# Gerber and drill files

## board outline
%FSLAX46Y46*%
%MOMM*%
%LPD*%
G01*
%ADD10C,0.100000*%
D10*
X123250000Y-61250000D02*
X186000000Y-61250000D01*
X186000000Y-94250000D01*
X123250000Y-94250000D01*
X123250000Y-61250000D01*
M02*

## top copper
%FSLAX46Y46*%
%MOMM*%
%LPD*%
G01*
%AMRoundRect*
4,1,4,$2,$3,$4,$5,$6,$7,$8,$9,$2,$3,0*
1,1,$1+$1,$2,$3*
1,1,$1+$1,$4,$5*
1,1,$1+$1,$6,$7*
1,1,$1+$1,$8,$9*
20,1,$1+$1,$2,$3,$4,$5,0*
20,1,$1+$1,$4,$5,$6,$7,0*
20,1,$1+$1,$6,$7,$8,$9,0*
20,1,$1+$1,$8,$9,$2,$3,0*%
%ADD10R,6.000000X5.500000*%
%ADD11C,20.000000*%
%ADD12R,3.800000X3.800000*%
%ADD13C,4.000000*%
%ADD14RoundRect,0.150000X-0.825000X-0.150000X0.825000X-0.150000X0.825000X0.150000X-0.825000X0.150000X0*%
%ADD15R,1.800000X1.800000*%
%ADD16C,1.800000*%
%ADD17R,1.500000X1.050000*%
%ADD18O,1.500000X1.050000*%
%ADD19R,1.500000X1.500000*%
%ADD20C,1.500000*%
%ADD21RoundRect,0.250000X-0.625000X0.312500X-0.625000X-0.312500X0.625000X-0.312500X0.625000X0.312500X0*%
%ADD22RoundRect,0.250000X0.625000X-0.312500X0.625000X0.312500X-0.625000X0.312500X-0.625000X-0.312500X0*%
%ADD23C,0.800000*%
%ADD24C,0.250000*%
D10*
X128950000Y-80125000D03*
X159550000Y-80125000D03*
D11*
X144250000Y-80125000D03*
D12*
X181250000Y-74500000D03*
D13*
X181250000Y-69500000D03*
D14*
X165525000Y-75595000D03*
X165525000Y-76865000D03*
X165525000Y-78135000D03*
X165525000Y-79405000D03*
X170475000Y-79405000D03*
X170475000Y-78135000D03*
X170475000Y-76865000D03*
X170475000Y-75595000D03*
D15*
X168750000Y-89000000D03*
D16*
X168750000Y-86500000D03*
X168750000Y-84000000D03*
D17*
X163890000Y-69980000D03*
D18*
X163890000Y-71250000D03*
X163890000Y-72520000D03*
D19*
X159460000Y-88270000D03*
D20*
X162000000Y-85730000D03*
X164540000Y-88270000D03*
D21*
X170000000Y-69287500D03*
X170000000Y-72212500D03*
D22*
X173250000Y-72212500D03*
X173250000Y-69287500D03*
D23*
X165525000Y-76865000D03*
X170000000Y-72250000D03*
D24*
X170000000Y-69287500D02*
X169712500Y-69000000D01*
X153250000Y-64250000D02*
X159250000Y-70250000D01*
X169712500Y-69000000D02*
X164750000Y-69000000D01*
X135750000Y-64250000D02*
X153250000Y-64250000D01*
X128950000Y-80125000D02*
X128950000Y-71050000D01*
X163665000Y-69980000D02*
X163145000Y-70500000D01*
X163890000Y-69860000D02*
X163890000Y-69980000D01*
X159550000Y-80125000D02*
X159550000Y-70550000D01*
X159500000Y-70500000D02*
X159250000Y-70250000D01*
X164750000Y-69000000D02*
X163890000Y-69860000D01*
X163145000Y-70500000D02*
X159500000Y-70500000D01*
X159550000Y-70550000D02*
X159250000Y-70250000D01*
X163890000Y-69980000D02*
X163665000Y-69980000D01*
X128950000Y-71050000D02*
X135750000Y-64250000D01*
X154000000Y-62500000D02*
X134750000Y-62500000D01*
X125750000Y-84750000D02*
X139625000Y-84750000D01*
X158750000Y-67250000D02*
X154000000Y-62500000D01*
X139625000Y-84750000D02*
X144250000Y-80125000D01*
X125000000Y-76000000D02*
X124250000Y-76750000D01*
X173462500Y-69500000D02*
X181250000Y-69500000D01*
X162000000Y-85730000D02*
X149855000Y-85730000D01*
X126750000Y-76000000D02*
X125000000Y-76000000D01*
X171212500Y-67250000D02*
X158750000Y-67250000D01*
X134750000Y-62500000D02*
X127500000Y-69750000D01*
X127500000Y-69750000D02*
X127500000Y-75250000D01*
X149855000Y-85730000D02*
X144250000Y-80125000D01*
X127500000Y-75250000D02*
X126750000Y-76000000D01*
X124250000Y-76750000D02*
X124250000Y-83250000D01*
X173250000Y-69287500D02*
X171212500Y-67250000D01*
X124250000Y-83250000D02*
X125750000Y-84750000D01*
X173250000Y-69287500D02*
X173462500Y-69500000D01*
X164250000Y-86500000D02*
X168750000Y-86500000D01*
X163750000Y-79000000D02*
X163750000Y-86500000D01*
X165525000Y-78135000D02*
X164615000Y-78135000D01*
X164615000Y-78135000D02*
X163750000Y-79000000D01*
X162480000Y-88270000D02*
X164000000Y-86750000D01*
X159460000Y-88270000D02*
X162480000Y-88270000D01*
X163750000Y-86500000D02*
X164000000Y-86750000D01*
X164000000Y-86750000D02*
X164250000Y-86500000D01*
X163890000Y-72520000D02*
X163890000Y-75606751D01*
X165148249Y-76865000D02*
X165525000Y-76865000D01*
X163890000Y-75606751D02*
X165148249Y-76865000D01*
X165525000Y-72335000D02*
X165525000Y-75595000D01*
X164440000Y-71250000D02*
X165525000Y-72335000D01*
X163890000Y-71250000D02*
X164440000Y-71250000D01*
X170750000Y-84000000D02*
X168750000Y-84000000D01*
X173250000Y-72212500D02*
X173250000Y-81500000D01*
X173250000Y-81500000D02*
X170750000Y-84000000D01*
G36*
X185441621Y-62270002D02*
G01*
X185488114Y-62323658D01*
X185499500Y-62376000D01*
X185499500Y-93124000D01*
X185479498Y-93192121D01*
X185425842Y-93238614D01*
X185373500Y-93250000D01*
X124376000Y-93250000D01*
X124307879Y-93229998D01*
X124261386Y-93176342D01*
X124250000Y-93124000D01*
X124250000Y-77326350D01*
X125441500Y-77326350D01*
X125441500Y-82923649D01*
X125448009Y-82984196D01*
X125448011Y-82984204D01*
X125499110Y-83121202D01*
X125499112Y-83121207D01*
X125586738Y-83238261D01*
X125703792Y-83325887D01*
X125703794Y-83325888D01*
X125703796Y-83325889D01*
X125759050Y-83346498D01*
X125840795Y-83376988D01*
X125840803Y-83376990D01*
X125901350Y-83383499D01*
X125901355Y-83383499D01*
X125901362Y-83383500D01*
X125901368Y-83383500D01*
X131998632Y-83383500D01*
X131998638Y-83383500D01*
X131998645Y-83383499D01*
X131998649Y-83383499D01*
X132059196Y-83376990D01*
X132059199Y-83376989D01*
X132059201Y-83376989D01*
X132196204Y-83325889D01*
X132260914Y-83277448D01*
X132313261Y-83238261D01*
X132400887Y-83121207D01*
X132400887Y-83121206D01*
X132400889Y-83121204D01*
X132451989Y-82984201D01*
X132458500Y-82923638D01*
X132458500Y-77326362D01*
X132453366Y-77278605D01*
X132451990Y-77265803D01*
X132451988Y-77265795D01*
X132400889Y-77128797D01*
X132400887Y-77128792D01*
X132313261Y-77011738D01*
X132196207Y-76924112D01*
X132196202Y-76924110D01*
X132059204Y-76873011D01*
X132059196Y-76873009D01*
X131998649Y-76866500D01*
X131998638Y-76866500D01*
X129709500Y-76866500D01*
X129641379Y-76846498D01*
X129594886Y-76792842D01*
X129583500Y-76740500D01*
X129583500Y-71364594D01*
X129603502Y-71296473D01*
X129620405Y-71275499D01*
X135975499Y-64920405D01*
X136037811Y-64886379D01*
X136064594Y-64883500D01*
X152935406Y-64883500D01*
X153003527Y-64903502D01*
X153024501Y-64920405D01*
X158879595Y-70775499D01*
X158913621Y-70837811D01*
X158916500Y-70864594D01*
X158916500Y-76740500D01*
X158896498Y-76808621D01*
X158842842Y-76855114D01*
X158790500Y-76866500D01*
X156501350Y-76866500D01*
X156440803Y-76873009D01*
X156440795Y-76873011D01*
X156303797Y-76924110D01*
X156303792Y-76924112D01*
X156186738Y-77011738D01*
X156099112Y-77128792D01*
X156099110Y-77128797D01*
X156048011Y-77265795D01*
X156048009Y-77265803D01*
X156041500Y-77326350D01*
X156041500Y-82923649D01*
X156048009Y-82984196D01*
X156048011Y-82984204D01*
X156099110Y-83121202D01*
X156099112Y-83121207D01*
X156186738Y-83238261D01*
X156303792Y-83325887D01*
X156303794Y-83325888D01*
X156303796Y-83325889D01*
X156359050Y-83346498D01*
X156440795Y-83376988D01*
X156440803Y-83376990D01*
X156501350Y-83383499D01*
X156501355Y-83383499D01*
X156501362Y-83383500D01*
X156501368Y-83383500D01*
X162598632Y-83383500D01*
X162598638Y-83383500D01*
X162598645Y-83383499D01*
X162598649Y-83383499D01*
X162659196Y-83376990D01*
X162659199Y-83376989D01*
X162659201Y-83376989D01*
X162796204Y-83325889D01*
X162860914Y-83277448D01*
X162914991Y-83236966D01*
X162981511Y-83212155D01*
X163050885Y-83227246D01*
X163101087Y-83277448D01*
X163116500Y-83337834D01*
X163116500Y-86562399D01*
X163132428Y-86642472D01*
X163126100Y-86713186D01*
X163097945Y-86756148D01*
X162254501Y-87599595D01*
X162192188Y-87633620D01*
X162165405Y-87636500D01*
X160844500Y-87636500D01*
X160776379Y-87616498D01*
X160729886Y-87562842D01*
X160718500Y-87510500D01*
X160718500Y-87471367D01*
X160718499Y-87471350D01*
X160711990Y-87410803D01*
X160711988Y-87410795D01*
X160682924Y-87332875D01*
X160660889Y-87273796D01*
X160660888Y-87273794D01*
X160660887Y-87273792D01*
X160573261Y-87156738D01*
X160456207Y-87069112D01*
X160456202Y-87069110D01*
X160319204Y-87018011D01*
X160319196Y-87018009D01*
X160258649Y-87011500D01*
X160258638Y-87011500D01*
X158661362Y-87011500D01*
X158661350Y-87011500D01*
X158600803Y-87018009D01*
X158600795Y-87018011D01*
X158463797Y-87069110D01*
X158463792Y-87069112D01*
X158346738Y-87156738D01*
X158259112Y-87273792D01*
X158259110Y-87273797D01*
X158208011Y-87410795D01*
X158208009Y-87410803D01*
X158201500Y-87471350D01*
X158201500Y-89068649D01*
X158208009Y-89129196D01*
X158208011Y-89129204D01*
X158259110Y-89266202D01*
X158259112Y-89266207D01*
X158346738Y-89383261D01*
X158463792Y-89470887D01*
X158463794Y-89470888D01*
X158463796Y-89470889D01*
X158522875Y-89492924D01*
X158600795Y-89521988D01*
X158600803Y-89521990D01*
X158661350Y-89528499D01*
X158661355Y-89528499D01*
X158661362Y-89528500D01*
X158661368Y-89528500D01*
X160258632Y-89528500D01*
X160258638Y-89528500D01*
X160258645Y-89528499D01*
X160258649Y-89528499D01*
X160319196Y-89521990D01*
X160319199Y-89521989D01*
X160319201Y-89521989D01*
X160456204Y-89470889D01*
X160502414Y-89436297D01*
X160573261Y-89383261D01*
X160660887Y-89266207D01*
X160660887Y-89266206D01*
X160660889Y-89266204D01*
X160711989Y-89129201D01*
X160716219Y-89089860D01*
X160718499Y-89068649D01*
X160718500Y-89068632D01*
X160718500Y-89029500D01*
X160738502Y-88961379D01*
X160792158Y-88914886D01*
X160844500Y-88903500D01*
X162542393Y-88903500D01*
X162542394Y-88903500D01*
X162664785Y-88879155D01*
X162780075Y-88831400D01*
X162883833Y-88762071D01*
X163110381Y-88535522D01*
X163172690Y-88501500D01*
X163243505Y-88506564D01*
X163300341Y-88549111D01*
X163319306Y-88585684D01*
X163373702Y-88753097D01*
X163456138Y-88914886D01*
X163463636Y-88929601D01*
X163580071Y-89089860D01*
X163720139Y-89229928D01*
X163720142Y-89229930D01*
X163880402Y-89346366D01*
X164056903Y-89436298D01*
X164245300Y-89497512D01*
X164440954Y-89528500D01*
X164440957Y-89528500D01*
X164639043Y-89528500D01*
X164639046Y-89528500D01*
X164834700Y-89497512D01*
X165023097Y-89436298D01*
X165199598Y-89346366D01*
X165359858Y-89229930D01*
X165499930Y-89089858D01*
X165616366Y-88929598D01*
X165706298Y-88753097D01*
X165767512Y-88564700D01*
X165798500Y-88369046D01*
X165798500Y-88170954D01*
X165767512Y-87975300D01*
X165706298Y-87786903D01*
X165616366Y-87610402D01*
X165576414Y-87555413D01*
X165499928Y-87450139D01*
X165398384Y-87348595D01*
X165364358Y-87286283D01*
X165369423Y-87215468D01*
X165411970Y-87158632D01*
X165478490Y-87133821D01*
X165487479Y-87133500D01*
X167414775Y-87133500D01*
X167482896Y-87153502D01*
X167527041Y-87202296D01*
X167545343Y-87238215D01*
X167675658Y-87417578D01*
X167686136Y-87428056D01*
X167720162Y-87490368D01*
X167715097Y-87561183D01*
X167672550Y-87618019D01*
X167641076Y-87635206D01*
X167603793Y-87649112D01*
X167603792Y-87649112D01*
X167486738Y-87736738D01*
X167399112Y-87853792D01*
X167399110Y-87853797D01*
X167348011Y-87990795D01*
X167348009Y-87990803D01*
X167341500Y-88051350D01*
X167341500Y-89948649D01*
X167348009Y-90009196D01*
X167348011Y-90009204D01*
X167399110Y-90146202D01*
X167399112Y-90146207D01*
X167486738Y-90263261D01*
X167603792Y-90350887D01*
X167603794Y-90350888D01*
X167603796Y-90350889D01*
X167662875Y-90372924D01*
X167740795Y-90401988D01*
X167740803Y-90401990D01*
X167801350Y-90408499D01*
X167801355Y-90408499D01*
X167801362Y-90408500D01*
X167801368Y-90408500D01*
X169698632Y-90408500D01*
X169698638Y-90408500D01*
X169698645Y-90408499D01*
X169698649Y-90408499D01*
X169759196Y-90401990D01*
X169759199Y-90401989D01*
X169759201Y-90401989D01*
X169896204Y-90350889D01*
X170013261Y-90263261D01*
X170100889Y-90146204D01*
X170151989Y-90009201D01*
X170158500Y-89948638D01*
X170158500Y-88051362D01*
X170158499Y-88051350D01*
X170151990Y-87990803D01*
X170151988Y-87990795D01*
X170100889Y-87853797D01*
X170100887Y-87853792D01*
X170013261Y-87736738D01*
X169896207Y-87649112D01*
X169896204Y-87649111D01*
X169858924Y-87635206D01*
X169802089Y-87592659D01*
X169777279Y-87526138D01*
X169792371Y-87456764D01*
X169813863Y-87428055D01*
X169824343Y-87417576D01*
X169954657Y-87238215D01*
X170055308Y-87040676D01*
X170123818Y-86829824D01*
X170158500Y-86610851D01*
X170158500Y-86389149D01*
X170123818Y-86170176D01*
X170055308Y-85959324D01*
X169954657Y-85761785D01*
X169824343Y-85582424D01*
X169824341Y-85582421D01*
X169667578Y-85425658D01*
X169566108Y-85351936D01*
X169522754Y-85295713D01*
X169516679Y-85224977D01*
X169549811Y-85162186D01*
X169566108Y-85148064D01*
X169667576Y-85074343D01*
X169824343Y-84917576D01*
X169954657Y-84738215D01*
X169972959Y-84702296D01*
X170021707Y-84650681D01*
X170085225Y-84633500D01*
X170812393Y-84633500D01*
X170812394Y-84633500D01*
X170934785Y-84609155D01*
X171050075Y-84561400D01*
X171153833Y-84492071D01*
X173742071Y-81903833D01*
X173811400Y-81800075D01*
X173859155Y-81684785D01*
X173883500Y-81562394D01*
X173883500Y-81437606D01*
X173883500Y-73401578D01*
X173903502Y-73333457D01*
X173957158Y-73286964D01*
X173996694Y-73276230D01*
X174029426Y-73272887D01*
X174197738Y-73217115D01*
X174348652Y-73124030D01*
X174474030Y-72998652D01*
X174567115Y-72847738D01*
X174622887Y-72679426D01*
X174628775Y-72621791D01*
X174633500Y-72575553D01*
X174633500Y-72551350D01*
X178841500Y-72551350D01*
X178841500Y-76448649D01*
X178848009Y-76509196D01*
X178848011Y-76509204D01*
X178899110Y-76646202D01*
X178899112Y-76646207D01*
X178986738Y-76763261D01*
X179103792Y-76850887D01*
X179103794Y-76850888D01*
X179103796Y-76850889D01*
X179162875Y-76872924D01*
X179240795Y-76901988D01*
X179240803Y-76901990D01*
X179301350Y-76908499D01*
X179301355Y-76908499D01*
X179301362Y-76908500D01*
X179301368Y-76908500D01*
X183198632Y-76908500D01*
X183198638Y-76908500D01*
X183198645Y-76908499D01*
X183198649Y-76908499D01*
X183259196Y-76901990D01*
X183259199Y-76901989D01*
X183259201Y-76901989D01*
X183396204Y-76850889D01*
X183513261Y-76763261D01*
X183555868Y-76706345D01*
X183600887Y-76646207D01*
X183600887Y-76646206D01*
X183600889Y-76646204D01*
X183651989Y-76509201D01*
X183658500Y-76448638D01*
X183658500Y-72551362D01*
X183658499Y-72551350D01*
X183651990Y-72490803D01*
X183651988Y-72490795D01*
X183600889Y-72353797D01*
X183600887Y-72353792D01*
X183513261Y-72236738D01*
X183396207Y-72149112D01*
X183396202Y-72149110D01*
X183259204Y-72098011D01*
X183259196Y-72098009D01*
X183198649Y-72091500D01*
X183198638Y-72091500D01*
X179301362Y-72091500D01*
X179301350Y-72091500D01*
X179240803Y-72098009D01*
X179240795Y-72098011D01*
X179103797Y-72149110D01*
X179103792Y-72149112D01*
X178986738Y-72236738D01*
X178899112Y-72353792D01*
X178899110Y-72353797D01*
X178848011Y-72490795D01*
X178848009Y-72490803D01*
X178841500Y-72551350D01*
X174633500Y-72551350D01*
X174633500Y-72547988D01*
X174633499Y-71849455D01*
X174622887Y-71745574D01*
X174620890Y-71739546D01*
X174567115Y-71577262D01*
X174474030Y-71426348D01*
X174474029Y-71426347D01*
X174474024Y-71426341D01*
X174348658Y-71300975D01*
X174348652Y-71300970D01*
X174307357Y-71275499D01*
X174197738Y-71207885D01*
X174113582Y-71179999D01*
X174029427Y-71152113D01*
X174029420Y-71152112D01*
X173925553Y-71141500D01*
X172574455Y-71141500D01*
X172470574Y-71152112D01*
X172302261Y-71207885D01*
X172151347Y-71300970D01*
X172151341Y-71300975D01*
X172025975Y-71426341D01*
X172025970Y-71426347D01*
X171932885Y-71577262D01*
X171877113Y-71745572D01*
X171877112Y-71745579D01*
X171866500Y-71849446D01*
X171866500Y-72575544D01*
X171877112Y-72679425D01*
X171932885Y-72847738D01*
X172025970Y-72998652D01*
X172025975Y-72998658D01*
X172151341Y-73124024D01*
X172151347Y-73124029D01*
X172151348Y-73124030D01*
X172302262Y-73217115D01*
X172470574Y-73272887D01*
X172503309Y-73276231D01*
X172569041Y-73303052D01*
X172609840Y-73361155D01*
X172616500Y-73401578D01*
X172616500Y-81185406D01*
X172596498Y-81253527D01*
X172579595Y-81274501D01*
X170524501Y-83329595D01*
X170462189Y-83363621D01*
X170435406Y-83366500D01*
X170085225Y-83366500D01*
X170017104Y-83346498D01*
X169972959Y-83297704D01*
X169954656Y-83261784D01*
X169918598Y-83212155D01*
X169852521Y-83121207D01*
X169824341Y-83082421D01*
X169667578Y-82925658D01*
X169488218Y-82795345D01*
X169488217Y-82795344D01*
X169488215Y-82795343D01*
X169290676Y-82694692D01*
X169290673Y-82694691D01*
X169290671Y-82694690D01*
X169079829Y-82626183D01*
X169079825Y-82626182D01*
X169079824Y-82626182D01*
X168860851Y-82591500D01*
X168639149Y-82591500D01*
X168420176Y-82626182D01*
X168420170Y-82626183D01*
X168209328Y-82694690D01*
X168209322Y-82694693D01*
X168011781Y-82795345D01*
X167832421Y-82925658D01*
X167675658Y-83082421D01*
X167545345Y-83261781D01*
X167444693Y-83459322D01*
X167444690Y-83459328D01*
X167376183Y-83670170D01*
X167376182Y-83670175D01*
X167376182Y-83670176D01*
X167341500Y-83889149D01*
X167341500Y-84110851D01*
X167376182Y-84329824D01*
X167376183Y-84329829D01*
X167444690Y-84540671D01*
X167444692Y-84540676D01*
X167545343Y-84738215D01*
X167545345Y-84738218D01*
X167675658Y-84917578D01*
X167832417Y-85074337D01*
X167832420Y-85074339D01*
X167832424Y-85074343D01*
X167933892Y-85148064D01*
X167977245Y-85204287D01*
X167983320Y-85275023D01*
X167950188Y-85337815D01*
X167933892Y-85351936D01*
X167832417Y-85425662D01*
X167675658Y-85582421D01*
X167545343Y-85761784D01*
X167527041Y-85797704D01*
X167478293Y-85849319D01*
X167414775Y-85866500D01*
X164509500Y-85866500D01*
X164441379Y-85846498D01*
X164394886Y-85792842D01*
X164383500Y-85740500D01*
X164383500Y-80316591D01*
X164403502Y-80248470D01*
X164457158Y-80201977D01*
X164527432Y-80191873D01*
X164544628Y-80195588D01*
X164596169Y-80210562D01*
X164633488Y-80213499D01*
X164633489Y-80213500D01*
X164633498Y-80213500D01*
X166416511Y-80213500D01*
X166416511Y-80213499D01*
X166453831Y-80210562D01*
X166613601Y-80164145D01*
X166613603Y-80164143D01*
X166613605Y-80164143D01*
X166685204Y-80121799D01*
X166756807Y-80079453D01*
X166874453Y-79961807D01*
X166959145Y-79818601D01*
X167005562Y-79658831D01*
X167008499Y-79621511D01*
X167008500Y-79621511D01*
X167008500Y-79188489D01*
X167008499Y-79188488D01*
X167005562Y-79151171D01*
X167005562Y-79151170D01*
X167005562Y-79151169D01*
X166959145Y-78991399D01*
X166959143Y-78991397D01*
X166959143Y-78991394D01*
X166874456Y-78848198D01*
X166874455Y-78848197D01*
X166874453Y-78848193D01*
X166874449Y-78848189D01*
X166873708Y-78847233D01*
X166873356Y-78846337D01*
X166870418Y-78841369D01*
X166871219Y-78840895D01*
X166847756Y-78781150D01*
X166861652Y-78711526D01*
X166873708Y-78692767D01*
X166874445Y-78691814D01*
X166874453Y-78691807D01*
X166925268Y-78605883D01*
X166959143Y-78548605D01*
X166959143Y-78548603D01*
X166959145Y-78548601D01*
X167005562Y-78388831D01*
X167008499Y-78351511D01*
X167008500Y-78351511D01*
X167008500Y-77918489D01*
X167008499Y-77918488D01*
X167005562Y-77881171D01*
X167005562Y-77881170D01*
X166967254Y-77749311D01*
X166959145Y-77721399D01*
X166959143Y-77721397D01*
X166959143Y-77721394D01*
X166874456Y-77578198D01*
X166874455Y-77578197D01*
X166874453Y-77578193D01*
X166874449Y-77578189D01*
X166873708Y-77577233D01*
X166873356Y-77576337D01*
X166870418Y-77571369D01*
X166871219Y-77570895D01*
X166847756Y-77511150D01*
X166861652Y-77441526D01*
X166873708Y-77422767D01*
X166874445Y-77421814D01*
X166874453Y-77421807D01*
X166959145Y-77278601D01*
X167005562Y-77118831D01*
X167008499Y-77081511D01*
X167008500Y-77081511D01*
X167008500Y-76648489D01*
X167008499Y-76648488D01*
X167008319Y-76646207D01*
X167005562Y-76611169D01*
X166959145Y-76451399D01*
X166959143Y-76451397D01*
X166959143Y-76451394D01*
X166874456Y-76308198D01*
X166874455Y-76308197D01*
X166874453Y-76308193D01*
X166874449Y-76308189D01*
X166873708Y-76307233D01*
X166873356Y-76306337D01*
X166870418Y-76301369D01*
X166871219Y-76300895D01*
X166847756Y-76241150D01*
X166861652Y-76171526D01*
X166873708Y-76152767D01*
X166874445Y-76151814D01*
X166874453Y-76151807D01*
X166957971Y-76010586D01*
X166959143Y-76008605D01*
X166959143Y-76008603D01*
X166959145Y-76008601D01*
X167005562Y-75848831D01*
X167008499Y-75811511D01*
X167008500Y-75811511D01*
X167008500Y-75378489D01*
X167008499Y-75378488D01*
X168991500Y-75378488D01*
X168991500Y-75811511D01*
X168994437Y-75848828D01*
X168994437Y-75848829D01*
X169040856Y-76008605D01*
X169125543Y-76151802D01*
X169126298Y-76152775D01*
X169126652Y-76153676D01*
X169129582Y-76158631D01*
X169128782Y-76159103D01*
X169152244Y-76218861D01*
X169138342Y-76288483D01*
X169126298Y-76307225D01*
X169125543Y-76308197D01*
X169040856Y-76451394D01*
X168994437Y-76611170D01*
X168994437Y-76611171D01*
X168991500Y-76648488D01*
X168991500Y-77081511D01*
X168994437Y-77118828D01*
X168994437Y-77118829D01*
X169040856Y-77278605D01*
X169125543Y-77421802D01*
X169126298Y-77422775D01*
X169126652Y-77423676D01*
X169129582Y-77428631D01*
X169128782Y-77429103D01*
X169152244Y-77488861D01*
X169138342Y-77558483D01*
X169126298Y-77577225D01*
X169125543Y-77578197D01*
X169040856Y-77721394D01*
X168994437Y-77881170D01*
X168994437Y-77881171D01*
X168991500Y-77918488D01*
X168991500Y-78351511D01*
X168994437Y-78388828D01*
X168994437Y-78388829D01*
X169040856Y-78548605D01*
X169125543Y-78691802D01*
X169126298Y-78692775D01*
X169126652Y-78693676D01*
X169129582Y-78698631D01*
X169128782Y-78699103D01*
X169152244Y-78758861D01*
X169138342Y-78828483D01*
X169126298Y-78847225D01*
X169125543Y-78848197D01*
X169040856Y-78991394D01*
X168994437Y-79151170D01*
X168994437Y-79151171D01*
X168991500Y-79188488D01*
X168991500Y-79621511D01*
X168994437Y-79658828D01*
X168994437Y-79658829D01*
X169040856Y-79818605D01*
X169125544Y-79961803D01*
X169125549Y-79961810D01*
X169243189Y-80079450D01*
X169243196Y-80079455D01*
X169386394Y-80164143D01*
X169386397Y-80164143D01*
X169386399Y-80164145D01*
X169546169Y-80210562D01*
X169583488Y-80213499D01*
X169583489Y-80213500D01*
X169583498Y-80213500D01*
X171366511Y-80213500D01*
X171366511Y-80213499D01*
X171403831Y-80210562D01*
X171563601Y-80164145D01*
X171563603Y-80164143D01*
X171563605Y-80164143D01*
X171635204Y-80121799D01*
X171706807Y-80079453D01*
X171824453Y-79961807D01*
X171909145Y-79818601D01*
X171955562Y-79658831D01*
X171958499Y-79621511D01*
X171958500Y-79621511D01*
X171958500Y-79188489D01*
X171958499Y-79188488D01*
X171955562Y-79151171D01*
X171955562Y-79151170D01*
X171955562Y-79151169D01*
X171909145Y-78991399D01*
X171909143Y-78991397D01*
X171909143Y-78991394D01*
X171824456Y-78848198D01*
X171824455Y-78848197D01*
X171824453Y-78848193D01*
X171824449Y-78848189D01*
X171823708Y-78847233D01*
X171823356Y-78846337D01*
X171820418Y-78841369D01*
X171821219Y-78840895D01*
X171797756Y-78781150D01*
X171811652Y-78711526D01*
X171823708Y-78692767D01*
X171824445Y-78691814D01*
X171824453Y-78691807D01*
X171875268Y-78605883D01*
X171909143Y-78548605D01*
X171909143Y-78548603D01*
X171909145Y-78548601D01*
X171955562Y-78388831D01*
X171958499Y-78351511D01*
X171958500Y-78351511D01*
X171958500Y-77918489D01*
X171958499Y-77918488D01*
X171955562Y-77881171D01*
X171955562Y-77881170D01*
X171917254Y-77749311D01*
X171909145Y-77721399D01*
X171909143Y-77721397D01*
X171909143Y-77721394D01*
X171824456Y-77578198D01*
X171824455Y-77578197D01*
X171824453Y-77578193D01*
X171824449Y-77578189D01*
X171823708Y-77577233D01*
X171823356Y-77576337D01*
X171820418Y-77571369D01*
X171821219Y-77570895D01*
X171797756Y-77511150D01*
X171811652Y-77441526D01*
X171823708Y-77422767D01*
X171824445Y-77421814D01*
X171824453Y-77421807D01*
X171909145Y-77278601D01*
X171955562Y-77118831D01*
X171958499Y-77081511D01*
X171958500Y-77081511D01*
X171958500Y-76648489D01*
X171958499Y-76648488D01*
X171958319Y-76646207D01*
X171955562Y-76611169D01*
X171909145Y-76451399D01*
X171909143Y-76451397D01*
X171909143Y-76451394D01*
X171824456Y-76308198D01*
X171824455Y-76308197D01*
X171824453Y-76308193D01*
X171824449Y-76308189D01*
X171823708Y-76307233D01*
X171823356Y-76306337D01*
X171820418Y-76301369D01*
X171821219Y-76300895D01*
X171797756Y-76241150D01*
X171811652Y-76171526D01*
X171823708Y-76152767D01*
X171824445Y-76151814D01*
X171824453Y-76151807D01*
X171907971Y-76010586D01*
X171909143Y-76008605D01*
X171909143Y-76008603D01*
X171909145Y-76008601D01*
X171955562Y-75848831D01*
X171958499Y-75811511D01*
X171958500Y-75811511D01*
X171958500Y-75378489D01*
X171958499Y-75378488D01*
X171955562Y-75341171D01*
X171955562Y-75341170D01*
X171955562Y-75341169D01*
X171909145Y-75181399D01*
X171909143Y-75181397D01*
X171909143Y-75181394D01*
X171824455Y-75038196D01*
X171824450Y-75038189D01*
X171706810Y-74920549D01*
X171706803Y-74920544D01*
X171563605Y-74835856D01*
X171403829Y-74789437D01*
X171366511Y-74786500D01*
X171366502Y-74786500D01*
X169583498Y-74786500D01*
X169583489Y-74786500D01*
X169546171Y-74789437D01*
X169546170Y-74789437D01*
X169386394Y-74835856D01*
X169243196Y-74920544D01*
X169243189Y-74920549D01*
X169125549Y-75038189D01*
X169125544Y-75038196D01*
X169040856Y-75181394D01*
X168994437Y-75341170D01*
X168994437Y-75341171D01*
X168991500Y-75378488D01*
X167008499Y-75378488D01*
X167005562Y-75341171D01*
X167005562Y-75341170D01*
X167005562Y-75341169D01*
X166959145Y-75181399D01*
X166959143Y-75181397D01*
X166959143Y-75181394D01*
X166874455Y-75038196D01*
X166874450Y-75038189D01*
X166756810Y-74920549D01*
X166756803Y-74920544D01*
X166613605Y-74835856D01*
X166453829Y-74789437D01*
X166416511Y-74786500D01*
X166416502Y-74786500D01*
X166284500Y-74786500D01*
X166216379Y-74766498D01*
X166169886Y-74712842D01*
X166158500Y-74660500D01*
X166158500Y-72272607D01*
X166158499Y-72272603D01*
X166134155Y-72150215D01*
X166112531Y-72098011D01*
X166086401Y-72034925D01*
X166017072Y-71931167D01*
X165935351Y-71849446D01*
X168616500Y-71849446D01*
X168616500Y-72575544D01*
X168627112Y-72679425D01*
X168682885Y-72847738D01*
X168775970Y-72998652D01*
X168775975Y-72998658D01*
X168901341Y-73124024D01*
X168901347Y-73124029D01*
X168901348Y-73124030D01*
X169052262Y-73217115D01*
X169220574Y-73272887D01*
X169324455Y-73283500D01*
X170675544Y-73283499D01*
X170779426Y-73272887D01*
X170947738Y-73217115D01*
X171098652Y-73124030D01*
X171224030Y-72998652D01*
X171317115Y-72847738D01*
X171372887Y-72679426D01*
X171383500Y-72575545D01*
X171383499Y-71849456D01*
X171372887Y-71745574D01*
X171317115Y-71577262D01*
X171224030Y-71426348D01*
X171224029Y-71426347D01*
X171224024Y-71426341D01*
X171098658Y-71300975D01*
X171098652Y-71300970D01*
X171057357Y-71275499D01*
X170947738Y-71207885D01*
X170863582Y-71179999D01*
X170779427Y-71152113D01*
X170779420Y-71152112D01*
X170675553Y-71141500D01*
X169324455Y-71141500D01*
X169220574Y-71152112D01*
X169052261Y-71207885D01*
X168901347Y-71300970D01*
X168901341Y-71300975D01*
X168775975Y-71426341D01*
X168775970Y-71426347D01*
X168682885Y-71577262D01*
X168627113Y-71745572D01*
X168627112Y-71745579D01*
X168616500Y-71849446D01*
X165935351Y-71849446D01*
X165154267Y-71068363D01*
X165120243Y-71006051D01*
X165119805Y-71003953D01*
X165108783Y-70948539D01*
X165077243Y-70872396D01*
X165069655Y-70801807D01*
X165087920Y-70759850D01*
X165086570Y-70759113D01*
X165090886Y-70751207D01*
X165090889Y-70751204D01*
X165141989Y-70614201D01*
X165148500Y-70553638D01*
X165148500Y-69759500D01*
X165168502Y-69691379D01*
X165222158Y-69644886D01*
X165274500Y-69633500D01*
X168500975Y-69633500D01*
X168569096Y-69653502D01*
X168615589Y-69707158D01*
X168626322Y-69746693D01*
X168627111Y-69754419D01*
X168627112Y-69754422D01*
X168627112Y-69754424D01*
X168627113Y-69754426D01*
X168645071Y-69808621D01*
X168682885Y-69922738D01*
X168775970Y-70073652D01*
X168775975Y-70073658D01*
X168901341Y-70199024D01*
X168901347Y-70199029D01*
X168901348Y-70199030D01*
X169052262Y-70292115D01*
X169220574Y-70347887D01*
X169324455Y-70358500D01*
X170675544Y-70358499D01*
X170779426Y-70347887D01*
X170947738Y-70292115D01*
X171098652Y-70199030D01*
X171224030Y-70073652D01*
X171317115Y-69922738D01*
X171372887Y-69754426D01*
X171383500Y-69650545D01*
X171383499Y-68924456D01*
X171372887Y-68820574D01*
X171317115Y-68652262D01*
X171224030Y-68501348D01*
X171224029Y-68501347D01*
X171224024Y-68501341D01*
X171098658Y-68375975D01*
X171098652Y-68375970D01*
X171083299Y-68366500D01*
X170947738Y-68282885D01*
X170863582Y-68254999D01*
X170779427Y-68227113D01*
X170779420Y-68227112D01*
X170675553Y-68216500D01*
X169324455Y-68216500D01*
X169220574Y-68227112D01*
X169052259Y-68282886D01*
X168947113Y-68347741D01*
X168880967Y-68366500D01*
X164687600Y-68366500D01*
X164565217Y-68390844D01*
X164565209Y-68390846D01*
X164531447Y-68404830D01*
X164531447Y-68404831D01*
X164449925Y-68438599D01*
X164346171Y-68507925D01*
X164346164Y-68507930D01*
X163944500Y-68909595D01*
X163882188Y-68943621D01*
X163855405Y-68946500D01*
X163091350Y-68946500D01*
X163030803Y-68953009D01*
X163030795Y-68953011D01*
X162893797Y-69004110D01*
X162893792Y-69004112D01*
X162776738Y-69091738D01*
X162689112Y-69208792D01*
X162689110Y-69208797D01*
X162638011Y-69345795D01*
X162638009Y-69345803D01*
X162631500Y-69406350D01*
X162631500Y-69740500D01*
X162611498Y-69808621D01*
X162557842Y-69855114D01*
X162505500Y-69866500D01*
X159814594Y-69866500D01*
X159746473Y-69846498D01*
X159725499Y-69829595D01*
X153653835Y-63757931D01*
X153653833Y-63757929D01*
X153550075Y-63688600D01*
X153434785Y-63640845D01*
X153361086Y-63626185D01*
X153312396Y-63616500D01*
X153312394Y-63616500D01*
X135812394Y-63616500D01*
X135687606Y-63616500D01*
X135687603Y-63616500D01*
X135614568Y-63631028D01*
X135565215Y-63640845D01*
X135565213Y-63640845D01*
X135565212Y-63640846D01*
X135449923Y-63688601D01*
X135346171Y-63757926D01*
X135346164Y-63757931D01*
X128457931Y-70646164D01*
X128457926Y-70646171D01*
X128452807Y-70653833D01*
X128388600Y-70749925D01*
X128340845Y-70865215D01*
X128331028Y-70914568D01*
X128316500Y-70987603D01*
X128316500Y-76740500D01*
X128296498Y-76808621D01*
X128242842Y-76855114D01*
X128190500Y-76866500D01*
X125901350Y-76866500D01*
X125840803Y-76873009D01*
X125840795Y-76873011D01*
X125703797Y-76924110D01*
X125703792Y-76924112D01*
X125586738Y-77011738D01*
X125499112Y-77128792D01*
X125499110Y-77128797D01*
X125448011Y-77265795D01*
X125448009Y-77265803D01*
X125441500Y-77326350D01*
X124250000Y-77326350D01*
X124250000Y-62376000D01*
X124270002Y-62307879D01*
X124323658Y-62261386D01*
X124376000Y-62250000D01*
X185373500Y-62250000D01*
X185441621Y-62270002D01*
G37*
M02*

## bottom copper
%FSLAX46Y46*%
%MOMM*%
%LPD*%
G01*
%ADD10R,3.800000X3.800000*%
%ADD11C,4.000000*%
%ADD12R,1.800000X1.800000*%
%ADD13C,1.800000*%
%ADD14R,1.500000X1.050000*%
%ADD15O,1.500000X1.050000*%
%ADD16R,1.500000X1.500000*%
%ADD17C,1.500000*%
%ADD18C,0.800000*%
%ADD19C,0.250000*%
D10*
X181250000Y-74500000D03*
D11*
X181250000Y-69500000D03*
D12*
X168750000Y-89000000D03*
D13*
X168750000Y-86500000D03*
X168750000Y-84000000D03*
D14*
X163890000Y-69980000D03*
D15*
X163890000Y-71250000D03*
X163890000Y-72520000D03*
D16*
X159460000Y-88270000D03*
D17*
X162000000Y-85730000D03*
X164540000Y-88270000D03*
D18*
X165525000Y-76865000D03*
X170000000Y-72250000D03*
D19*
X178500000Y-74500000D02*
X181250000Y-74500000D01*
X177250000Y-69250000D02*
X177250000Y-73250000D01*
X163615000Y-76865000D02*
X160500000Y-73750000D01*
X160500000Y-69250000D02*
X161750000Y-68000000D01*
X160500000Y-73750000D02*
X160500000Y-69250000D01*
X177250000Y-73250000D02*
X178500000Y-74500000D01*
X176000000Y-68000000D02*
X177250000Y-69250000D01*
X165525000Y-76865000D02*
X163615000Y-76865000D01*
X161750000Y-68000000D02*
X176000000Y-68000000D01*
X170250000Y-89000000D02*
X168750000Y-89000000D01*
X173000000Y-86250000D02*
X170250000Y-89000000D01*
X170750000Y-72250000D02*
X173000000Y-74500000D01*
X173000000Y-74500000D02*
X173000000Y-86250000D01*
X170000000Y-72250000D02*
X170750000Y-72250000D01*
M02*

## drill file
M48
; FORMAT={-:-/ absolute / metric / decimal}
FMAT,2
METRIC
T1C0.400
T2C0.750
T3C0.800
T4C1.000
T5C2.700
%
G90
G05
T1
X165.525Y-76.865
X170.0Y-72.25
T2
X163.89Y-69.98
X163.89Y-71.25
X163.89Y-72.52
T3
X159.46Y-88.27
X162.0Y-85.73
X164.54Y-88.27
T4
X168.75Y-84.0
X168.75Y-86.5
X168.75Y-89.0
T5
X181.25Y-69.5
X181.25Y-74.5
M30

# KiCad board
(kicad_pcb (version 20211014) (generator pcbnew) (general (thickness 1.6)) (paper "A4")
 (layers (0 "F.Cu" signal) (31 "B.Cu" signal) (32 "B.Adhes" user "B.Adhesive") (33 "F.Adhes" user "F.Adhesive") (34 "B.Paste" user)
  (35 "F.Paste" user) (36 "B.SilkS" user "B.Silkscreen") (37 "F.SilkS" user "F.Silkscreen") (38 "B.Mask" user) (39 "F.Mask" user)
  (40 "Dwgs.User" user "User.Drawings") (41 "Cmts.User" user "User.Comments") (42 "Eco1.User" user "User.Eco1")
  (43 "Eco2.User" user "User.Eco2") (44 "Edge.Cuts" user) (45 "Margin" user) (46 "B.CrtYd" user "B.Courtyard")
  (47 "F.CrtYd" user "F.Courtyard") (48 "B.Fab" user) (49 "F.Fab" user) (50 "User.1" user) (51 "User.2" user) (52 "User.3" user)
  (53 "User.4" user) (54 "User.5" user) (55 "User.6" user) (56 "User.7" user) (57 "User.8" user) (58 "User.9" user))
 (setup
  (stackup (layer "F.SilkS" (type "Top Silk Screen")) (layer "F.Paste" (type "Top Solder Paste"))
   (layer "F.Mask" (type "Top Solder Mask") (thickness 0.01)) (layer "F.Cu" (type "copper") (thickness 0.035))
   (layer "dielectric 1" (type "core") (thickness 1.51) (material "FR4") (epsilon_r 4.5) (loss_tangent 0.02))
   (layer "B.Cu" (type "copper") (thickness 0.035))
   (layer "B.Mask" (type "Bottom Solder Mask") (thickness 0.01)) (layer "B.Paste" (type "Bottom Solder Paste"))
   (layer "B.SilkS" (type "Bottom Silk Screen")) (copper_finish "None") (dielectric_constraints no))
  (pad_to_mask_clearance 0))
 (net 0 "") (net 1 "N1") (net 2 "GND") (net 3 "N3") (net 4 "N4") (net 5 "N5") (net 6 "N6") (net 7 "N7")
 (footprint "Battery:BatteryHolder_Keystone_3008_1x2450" (layer "F.Cu") (at 144.25 80.125)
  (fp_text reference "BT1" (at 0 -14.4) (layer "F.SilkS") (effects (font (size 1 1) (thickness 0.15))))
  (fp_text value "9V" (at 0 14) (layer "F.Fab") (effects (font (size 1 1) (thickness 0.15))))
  (pad "1" smd rect (at -15.3 0) (size 6 5.5) (layers "F.Cu" "F.Paste" "F.Mask") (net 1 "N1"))
  (pad "1" smd rect (at 15.3 0) (size 6 5.5) (layers "F.Cu" "F.Paste" "F.Mask") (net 1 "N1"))
  (pad "2" smd circle (at 0 0) (size 20 20) (layers "F.Cu" "F.Mask") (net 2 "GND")))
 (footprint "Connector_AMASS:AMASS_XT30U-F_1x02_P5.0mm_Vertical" (layer "F.Cu") (at 181.25 74.5 90)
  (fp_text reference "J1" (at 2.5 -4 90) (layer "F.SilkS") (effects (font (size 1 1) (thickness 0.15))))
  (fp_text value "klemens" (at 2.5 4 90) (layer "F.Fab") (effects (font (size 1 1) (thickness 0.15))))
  (pad "1" thru_hole rect (at 0 0 90) (size 3.8 3.8) (drill 2.7) (layers *.Cu *.Mask) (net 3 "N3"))
  (pad "2" thru_hole circle (at 5 0 90) (size 4 4) (drill 2.7) (layers *.Cu *.Mask) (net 2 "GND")))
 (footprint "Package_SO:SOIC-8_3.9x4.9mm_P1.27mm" (layer "F.Cu") (at 168 77.5)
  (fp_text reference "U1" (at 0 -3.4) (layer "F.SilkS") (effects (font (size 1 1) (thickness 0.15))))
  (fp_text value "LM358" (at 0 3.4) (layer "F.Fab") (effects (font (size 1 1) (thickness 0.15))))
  (pad "1" smd roundrect (at -2.475 -1.905) (size 1.95 0.6) (layers "F.Cu" "F.Paste" "F.Mask") (roundrect_rratio 0.25) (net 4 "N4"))
  (pad "2" smd roundrect (at -2.475 -0.635) (size 1.95 0.6) (layers "F.Cu" "F.Paste" "F.Mask") (roundrect_rratio 0.25) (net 3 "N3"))
  (pad "3" smd roundrect (at -2.475 0.635) (size 1.95 0.6) (layers "F.Cu" "F.Paste" "F.Mask") (roundrect_rratio 0.25) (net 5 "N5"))
  (pad "4" smd roundrect (at -2.475 1.905) (size 1.95 0.6) (layers "F.Cu" "F.Paste" "F.Mask") (roundrect_rratio 0.25))
  (pad "5" smd roundrect (at 2.475 1.905) (size 1.95 0.6) (layers "F.Cu" "F.Paste" "F.Mask") (roundrect_rratio 0.25))
  (pad "6" smd roundrect (at 2.475 0.635) (size 1.95 0.6) (layers "F.Cu" "F.Paste" "F.Mask") (roundrect_rratio 0.25))
  (pad "7" smd roundrect (at 2.475 -0.635) (size 1.95 0.6) (layers "F.Cu" "F.Paste" "F.Mask") (roundrect_rratio 0.25))
  (pad "8" smd roundrect (at 2.475 -1.905) (size 1.95 0.6) (layers "F.Cu" "F.Paste" "F.Mask") (roundrect_rratio 0.25)))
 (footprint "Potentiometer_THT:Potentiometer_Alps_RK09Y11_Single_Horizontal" (layer "F.Cu") (at 168.75 89 180)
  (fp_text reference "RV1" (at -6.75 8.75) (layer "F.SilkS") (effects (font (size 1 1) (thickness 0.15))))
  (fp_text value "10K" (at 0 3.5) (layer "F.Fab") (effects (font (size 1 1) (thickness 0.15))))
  (pad "1" thru_hole rect (at 0 0) (size 1.8 1.8) (drill 1) (layers *.Cu *.Mask) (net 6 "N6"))
  (pad "2" thru_hole circle (at 0 2.5) (size 1.8 1.8) (drill 1) (layers *.Cu *.Mask) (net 5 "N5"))
  (pad "3" thru_hole circle (at 0 5) (size 1.8 1.8) (drill 1) (layers *.Cu *.Mask) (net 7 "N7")))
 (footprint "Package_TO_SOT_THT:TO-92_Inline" (layer "F.Cu") (at 163.89 69.98 -90)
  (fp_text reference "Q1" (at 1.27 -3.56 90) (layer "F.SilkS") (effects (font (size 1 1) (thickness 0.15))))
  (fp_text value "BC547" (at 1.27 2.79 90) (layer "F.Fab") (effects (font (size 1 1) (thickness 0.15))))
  (pad "1" thru_hole rect (at 0 0 270) (size 1.05 1.5) (drill 0.75) (layers *.Cu *.Mask) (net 1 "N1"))
  (pad "2" thru_hole oval (at 1.27 0 270) (size 1.05 1.5) (drill 0.75) (layers *.Cu *.Mask) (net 4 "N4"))
  (pad "3" thru_hole oval (at 2.54 0 270) (size 1.05 1.5) (drill 0.75) (layers *.Cu *.Mask) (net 3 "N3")))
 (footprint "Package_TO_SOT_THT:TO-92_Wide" (layer "F.Cu") (at 159.46 88.27)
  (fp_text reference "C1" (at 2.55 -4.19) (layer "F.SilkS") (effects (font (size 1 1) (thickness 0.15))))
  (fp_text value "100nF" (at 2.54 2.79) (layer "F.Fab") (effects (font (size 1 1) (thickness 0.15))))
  (pad "1" thru_hole rect (at 0 0) (size 1.5 1.5) (drill 0.8) (layers *.Cu *.Mask) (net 5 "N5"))
  (pad "2" thru_hole circle (at 2.54 -2.54) (size 1.5 1.5) (drill 0.8) (layers *.Cu *.Mask) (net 2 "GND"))
  (pad "3" thru_hole circle (at 5.08 0) (size 1.5 1.5) (drill 0.8) (layers *.Cu *.Mask)))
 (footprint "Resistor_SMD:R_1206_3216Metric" (layer "F.Cu") (at 170 70.75 -90)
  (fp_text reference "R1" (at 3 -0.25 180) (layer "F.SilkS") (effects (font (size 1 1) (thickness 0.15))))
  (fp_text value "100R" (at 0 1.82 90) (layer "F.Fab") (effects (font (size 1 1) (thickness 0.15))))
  (pad "1" smd roundrect (at -1.4625 0 270) (size 1.125 1.75) (layers "F.Cu" "F.Paste" "F.Mask") (roundrect_rratio 0.2222222222)
   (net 1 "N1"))
  (pad "2" smd roundrect (at 1.4625 0 270) (size 1.125 1.75) (layers "F.Cu" "F.Paste" "F.Mask") (roundrect_rratio 0.2222222222) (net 6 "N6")))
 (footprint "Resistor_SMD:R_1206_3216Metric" (layer "F.Cu") (at 173.25 70.75 90)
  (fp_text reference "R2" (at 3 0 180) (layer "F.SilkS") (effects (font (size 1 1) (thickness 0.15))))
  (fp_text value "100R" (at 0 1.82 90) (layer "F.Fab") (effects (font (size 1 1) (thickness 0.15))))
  (pad "1" smd roundrect (at -1.4625 0 90) (size 1.125 1.75) (layers "F.Cu" "F.Paste" "F.Mask") (roundrect_rratio 0.2222222222) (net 7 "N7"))
  (pad "2" smd roundrect (at 1.4625 0 90) (size 1.125 1.75) (layers "F.Cu" "F.Paste" "F.Mask") (roundrect_rratio 0.2222222222) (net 2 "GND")))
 (gr_rect (start 123.25 61.25) (end 186 94.25) (layer "Edge.Cuts") (width 0.1) (fill none))
 (segment (start 170 69.2875) (end 169.7125 69) (width 0.25) (layer "F.Cu") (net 1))
 (segment (start 153.25 64.25) (end 159.25 70.25) (width 0.25) (layer "F.Cu") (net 1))
 (segment (start 169.7125 69) (end 164.75 69) (width 0.25) (layer "F.Cu") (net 1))
 (segment (start 135.75 64.25) (end 153.25 64.25) (width 0.25) (layer "F.Cu") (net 1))
 (segment (start 128.95 80.125) (end 128.95 71.05) (width 0.25) (layer "F.Cu") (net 1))
 (segment (start 163.665 69.98) (end 163.145 70.5) (width 0.25) (layer "F.Cu") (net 1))
 (segment (start 163.89 69.86) (end 163.89 69.98) (width 0.25) (layer "F.Cu") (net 1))
 (segment (start 159.55 80.125) (end 159.55 70.55) (width 0.25) (layer "F.Cu") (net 1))
 (segment (start 159.5 70.5) (end 159.25 70.25) (width 0.25) (layer "F.Cu") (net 1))
 (segment (start 164.75 69) (end 163.89 69.86) (width 0.25) (layer "F.Cu") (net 1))
 (segment (start 163.145 70.5) (end 159.5 70.5) (width 0.25) (layer "F.Cu") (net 1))
 (segment (start 159.55 70.55) (end 159.25 70.25) (width 0.25) (layer "F.Cu") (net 1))
 (segment (start 163.89 69.98) (end 163.665 69.98) (width 0.25) (layer "F.Cu") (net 1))
 (segment (start 128.95 71.05) (end 135.75 64.25) (width 0.25) (layer "F.Cu") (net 1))
 (segment (start 154 62.5) (end 134.75 62.5) (width 0.25) (layer "F.Cu") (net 2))
 (segment (start 125.75 84.75) (end 139.625 84.75) (width 0.25) (layer "F.Cu") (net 2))
 (segment (start 158.75 67.25) (end 154 62.5) (width 0.25) (layer "F.Cu") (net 2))
 (segment (start 139.625 84.75) (end 144.25 80.125) (width 0.25) (layer "F.Cu") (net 2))
 (segment (start 125 76) (end 124.25 76.75) (width 0.25) (layer "F.Cu") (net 2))
 (segment (start 173.4625 69.5) (end 181.25 69.5) (width 0.25) (layer "F.Cu") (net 2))
 (segment (start 162 85.73) (end 149.855 85.73) (width 0.25) (layer "F.Cu") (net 2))
 (segment (start 126.75 76) (end 125 76) (width 0.25) (layer "F.Cu") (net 2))
 (segment (start 171.2125 67.25) (end 158.75 67.25) (width 0.25) (layer "F.Cu") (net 2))
 (segment (start 134.75 62.5) (end 127.5 69.75) (width 0.25) (layer "F.Cu") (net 2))
 (segment (start 127.5 69.75) (end 127.5 75.25) (width 0.25) (layer "F.Cu") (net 2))
 (segment (start 149.855 85.73) (end 144.25 80.125) (width 0.25) (layer "F.Cu") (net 2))
 (segment (start 127.5 75.25) (end 126.75 76) (width 0.25) (layer "F.Cu") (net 2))
 (segment (start 124.25 76.75) (end 124.25 83.25) (width 0.25) (layer "F.Cu") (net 2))
 (segment (start 173.25 69.2875) (end 171.2125 67.25) (width 0.25) (layer "F.Cu") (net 2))
 (segment (start 124.25 83.25) (end 125.75 84.75) (width 0.25) (layer "F.Cu") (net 2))
 (segment (start 173.25 69.2875) (end 173.4625 69.5) (width 0.25) (layer "F.Cu") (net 2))
 (segment (start 164.25 86.5) (end 168.75 86.5) (width 0.25) (layer "F.Cu") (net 5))
 (segment (start 163.75 79) (end 163.75 86.5) (width 0.25) (layer "F.Cu") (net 5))
 (segment (start 165.525 78.135) (end 164.615 78.135) (width 0.25) (layer "F.Cu") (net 5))
 (segment (start 164.615 78.135) (end 163.75 79) (width 0.25) (layer "F.Cu") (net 5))
 (segment (start 162.48 88.27) (end 164 86.75) (width 0.25) (layer "F.Cu") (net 5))
 (segment (start 159.46 88.27) (end 162.48 88.27) (width 0.25) (layer "F.Cu") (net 5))
 (segment (start 163.75 86.5) (end 164 86.75) (width 0.25) (layer "F.Cu") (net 5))
 (segment (start 164 86.75) (end 164.25 86.5) (width 0.25) (layer "F.Cu") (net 5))
 (segment (start 163.89 72.52) (end 163.89 75.606751) (width 0.25) (layer "F.Cu") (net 3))
 (segment (start 165.148249 76.865) (end 165.525 76.865) (width 0.25) (layer "F.Cu") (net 3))
 (segment (start 163.89 75.606751) (end 165.148249 76.865) (width 0.25) (layer "F.Cu") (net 3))
 (via (at 165.525 76.865) (size 0.8) (drill 0.4) (layers "F.Cu" "B.Cu") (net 3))
 (segment (start 178.5 74.5) (end 181.25 74.5) (width 0.25) (layer "B.Cu") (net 3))
 (segment (start 177.25 69.25) (end 177.25 73.25) (width 0.25) (layer "B.Cu") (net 3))
 (segment (start 163.615 76.865) (end 160.5 73.75) (width 0.25) (layer "B.Cu") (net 3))
 (segment (start 160.5 69.25) (end 161.75 68) (width 0.25) (layer "B.Cu") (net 3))
 (segment (start 160.5 73.75) (end 160.5 69.25) (width 0.25) (layer "B.Cu") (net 3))
 (segment (start 177.25 73.25) (end 178.5 74.5) (width 0.25) (layer "B.Cu") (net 3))
 (segment (start 176 68) (end 177.25 69.25) (width 0.25) (layer "B.Cu") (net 3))
 (segment (start 165.525 76.865) (end 163.615 76.865) (width 0.25) (layer "B.Cu") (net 3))
 (segment (start 161.75 68) (end 176 68) (width 0.25) (layer "B.Cu") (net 3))
 (segment (start 165.525 72.335) (end 165.525 75.595) (width 0.25) (layer "F.Cu") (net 4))
 (segment (start 164.44 71.25) (end 165.525 72.335) (width 0.25) (layer "F.Cu") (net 4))
 (segment (start 163.89 71.25) (end 164.44 71.25) (width 0.25) (layer "F.Cu") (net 4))
 (via (at 170 72.25) (size 0.8) (drill 0.4) (layers "F.Cu" "B.Cu") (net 6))
 (segment (start 170.25 89) (end 168.75 89) (width 0.25) (layer "B.Cu") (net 6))
 (segment (start 173 86.25) (end 170.25 89) (width 0.25) (layer "B.Cu") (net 6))
 (segment (start 170.75 72.25) (end 173 74.5) (width 0.25) (layer "B.Cu") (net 6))
 (segment (start 173 74.5) (end 173 86.25) (width 0.25) (layer "B.Cu") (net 6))
 (segment (start 170 72.25) (end 170.75 72.25) (width 0.25) (layer "B.Cu") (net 6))
 (segment (start 170.75 84) (end 168.75 84) (width 0.25) (layer "F.Cu") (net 7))
 (segment (start 173.25 72.2125) (end 173.25 81.5) (width 0.25) (layer "F.Cu") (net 7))
 (segment (start 173.25 81.5) (end 170.75 84) (width 0.25) (layer "F.Cu") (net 7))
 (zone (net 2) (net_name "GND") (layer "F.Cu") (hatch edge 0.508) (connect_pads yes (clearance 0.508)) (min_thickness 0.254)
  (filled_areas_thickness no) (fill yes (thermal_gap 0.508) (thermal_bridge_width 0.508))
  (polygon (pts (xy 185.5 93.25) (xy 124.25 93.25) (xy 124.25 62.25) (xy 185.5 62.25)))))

